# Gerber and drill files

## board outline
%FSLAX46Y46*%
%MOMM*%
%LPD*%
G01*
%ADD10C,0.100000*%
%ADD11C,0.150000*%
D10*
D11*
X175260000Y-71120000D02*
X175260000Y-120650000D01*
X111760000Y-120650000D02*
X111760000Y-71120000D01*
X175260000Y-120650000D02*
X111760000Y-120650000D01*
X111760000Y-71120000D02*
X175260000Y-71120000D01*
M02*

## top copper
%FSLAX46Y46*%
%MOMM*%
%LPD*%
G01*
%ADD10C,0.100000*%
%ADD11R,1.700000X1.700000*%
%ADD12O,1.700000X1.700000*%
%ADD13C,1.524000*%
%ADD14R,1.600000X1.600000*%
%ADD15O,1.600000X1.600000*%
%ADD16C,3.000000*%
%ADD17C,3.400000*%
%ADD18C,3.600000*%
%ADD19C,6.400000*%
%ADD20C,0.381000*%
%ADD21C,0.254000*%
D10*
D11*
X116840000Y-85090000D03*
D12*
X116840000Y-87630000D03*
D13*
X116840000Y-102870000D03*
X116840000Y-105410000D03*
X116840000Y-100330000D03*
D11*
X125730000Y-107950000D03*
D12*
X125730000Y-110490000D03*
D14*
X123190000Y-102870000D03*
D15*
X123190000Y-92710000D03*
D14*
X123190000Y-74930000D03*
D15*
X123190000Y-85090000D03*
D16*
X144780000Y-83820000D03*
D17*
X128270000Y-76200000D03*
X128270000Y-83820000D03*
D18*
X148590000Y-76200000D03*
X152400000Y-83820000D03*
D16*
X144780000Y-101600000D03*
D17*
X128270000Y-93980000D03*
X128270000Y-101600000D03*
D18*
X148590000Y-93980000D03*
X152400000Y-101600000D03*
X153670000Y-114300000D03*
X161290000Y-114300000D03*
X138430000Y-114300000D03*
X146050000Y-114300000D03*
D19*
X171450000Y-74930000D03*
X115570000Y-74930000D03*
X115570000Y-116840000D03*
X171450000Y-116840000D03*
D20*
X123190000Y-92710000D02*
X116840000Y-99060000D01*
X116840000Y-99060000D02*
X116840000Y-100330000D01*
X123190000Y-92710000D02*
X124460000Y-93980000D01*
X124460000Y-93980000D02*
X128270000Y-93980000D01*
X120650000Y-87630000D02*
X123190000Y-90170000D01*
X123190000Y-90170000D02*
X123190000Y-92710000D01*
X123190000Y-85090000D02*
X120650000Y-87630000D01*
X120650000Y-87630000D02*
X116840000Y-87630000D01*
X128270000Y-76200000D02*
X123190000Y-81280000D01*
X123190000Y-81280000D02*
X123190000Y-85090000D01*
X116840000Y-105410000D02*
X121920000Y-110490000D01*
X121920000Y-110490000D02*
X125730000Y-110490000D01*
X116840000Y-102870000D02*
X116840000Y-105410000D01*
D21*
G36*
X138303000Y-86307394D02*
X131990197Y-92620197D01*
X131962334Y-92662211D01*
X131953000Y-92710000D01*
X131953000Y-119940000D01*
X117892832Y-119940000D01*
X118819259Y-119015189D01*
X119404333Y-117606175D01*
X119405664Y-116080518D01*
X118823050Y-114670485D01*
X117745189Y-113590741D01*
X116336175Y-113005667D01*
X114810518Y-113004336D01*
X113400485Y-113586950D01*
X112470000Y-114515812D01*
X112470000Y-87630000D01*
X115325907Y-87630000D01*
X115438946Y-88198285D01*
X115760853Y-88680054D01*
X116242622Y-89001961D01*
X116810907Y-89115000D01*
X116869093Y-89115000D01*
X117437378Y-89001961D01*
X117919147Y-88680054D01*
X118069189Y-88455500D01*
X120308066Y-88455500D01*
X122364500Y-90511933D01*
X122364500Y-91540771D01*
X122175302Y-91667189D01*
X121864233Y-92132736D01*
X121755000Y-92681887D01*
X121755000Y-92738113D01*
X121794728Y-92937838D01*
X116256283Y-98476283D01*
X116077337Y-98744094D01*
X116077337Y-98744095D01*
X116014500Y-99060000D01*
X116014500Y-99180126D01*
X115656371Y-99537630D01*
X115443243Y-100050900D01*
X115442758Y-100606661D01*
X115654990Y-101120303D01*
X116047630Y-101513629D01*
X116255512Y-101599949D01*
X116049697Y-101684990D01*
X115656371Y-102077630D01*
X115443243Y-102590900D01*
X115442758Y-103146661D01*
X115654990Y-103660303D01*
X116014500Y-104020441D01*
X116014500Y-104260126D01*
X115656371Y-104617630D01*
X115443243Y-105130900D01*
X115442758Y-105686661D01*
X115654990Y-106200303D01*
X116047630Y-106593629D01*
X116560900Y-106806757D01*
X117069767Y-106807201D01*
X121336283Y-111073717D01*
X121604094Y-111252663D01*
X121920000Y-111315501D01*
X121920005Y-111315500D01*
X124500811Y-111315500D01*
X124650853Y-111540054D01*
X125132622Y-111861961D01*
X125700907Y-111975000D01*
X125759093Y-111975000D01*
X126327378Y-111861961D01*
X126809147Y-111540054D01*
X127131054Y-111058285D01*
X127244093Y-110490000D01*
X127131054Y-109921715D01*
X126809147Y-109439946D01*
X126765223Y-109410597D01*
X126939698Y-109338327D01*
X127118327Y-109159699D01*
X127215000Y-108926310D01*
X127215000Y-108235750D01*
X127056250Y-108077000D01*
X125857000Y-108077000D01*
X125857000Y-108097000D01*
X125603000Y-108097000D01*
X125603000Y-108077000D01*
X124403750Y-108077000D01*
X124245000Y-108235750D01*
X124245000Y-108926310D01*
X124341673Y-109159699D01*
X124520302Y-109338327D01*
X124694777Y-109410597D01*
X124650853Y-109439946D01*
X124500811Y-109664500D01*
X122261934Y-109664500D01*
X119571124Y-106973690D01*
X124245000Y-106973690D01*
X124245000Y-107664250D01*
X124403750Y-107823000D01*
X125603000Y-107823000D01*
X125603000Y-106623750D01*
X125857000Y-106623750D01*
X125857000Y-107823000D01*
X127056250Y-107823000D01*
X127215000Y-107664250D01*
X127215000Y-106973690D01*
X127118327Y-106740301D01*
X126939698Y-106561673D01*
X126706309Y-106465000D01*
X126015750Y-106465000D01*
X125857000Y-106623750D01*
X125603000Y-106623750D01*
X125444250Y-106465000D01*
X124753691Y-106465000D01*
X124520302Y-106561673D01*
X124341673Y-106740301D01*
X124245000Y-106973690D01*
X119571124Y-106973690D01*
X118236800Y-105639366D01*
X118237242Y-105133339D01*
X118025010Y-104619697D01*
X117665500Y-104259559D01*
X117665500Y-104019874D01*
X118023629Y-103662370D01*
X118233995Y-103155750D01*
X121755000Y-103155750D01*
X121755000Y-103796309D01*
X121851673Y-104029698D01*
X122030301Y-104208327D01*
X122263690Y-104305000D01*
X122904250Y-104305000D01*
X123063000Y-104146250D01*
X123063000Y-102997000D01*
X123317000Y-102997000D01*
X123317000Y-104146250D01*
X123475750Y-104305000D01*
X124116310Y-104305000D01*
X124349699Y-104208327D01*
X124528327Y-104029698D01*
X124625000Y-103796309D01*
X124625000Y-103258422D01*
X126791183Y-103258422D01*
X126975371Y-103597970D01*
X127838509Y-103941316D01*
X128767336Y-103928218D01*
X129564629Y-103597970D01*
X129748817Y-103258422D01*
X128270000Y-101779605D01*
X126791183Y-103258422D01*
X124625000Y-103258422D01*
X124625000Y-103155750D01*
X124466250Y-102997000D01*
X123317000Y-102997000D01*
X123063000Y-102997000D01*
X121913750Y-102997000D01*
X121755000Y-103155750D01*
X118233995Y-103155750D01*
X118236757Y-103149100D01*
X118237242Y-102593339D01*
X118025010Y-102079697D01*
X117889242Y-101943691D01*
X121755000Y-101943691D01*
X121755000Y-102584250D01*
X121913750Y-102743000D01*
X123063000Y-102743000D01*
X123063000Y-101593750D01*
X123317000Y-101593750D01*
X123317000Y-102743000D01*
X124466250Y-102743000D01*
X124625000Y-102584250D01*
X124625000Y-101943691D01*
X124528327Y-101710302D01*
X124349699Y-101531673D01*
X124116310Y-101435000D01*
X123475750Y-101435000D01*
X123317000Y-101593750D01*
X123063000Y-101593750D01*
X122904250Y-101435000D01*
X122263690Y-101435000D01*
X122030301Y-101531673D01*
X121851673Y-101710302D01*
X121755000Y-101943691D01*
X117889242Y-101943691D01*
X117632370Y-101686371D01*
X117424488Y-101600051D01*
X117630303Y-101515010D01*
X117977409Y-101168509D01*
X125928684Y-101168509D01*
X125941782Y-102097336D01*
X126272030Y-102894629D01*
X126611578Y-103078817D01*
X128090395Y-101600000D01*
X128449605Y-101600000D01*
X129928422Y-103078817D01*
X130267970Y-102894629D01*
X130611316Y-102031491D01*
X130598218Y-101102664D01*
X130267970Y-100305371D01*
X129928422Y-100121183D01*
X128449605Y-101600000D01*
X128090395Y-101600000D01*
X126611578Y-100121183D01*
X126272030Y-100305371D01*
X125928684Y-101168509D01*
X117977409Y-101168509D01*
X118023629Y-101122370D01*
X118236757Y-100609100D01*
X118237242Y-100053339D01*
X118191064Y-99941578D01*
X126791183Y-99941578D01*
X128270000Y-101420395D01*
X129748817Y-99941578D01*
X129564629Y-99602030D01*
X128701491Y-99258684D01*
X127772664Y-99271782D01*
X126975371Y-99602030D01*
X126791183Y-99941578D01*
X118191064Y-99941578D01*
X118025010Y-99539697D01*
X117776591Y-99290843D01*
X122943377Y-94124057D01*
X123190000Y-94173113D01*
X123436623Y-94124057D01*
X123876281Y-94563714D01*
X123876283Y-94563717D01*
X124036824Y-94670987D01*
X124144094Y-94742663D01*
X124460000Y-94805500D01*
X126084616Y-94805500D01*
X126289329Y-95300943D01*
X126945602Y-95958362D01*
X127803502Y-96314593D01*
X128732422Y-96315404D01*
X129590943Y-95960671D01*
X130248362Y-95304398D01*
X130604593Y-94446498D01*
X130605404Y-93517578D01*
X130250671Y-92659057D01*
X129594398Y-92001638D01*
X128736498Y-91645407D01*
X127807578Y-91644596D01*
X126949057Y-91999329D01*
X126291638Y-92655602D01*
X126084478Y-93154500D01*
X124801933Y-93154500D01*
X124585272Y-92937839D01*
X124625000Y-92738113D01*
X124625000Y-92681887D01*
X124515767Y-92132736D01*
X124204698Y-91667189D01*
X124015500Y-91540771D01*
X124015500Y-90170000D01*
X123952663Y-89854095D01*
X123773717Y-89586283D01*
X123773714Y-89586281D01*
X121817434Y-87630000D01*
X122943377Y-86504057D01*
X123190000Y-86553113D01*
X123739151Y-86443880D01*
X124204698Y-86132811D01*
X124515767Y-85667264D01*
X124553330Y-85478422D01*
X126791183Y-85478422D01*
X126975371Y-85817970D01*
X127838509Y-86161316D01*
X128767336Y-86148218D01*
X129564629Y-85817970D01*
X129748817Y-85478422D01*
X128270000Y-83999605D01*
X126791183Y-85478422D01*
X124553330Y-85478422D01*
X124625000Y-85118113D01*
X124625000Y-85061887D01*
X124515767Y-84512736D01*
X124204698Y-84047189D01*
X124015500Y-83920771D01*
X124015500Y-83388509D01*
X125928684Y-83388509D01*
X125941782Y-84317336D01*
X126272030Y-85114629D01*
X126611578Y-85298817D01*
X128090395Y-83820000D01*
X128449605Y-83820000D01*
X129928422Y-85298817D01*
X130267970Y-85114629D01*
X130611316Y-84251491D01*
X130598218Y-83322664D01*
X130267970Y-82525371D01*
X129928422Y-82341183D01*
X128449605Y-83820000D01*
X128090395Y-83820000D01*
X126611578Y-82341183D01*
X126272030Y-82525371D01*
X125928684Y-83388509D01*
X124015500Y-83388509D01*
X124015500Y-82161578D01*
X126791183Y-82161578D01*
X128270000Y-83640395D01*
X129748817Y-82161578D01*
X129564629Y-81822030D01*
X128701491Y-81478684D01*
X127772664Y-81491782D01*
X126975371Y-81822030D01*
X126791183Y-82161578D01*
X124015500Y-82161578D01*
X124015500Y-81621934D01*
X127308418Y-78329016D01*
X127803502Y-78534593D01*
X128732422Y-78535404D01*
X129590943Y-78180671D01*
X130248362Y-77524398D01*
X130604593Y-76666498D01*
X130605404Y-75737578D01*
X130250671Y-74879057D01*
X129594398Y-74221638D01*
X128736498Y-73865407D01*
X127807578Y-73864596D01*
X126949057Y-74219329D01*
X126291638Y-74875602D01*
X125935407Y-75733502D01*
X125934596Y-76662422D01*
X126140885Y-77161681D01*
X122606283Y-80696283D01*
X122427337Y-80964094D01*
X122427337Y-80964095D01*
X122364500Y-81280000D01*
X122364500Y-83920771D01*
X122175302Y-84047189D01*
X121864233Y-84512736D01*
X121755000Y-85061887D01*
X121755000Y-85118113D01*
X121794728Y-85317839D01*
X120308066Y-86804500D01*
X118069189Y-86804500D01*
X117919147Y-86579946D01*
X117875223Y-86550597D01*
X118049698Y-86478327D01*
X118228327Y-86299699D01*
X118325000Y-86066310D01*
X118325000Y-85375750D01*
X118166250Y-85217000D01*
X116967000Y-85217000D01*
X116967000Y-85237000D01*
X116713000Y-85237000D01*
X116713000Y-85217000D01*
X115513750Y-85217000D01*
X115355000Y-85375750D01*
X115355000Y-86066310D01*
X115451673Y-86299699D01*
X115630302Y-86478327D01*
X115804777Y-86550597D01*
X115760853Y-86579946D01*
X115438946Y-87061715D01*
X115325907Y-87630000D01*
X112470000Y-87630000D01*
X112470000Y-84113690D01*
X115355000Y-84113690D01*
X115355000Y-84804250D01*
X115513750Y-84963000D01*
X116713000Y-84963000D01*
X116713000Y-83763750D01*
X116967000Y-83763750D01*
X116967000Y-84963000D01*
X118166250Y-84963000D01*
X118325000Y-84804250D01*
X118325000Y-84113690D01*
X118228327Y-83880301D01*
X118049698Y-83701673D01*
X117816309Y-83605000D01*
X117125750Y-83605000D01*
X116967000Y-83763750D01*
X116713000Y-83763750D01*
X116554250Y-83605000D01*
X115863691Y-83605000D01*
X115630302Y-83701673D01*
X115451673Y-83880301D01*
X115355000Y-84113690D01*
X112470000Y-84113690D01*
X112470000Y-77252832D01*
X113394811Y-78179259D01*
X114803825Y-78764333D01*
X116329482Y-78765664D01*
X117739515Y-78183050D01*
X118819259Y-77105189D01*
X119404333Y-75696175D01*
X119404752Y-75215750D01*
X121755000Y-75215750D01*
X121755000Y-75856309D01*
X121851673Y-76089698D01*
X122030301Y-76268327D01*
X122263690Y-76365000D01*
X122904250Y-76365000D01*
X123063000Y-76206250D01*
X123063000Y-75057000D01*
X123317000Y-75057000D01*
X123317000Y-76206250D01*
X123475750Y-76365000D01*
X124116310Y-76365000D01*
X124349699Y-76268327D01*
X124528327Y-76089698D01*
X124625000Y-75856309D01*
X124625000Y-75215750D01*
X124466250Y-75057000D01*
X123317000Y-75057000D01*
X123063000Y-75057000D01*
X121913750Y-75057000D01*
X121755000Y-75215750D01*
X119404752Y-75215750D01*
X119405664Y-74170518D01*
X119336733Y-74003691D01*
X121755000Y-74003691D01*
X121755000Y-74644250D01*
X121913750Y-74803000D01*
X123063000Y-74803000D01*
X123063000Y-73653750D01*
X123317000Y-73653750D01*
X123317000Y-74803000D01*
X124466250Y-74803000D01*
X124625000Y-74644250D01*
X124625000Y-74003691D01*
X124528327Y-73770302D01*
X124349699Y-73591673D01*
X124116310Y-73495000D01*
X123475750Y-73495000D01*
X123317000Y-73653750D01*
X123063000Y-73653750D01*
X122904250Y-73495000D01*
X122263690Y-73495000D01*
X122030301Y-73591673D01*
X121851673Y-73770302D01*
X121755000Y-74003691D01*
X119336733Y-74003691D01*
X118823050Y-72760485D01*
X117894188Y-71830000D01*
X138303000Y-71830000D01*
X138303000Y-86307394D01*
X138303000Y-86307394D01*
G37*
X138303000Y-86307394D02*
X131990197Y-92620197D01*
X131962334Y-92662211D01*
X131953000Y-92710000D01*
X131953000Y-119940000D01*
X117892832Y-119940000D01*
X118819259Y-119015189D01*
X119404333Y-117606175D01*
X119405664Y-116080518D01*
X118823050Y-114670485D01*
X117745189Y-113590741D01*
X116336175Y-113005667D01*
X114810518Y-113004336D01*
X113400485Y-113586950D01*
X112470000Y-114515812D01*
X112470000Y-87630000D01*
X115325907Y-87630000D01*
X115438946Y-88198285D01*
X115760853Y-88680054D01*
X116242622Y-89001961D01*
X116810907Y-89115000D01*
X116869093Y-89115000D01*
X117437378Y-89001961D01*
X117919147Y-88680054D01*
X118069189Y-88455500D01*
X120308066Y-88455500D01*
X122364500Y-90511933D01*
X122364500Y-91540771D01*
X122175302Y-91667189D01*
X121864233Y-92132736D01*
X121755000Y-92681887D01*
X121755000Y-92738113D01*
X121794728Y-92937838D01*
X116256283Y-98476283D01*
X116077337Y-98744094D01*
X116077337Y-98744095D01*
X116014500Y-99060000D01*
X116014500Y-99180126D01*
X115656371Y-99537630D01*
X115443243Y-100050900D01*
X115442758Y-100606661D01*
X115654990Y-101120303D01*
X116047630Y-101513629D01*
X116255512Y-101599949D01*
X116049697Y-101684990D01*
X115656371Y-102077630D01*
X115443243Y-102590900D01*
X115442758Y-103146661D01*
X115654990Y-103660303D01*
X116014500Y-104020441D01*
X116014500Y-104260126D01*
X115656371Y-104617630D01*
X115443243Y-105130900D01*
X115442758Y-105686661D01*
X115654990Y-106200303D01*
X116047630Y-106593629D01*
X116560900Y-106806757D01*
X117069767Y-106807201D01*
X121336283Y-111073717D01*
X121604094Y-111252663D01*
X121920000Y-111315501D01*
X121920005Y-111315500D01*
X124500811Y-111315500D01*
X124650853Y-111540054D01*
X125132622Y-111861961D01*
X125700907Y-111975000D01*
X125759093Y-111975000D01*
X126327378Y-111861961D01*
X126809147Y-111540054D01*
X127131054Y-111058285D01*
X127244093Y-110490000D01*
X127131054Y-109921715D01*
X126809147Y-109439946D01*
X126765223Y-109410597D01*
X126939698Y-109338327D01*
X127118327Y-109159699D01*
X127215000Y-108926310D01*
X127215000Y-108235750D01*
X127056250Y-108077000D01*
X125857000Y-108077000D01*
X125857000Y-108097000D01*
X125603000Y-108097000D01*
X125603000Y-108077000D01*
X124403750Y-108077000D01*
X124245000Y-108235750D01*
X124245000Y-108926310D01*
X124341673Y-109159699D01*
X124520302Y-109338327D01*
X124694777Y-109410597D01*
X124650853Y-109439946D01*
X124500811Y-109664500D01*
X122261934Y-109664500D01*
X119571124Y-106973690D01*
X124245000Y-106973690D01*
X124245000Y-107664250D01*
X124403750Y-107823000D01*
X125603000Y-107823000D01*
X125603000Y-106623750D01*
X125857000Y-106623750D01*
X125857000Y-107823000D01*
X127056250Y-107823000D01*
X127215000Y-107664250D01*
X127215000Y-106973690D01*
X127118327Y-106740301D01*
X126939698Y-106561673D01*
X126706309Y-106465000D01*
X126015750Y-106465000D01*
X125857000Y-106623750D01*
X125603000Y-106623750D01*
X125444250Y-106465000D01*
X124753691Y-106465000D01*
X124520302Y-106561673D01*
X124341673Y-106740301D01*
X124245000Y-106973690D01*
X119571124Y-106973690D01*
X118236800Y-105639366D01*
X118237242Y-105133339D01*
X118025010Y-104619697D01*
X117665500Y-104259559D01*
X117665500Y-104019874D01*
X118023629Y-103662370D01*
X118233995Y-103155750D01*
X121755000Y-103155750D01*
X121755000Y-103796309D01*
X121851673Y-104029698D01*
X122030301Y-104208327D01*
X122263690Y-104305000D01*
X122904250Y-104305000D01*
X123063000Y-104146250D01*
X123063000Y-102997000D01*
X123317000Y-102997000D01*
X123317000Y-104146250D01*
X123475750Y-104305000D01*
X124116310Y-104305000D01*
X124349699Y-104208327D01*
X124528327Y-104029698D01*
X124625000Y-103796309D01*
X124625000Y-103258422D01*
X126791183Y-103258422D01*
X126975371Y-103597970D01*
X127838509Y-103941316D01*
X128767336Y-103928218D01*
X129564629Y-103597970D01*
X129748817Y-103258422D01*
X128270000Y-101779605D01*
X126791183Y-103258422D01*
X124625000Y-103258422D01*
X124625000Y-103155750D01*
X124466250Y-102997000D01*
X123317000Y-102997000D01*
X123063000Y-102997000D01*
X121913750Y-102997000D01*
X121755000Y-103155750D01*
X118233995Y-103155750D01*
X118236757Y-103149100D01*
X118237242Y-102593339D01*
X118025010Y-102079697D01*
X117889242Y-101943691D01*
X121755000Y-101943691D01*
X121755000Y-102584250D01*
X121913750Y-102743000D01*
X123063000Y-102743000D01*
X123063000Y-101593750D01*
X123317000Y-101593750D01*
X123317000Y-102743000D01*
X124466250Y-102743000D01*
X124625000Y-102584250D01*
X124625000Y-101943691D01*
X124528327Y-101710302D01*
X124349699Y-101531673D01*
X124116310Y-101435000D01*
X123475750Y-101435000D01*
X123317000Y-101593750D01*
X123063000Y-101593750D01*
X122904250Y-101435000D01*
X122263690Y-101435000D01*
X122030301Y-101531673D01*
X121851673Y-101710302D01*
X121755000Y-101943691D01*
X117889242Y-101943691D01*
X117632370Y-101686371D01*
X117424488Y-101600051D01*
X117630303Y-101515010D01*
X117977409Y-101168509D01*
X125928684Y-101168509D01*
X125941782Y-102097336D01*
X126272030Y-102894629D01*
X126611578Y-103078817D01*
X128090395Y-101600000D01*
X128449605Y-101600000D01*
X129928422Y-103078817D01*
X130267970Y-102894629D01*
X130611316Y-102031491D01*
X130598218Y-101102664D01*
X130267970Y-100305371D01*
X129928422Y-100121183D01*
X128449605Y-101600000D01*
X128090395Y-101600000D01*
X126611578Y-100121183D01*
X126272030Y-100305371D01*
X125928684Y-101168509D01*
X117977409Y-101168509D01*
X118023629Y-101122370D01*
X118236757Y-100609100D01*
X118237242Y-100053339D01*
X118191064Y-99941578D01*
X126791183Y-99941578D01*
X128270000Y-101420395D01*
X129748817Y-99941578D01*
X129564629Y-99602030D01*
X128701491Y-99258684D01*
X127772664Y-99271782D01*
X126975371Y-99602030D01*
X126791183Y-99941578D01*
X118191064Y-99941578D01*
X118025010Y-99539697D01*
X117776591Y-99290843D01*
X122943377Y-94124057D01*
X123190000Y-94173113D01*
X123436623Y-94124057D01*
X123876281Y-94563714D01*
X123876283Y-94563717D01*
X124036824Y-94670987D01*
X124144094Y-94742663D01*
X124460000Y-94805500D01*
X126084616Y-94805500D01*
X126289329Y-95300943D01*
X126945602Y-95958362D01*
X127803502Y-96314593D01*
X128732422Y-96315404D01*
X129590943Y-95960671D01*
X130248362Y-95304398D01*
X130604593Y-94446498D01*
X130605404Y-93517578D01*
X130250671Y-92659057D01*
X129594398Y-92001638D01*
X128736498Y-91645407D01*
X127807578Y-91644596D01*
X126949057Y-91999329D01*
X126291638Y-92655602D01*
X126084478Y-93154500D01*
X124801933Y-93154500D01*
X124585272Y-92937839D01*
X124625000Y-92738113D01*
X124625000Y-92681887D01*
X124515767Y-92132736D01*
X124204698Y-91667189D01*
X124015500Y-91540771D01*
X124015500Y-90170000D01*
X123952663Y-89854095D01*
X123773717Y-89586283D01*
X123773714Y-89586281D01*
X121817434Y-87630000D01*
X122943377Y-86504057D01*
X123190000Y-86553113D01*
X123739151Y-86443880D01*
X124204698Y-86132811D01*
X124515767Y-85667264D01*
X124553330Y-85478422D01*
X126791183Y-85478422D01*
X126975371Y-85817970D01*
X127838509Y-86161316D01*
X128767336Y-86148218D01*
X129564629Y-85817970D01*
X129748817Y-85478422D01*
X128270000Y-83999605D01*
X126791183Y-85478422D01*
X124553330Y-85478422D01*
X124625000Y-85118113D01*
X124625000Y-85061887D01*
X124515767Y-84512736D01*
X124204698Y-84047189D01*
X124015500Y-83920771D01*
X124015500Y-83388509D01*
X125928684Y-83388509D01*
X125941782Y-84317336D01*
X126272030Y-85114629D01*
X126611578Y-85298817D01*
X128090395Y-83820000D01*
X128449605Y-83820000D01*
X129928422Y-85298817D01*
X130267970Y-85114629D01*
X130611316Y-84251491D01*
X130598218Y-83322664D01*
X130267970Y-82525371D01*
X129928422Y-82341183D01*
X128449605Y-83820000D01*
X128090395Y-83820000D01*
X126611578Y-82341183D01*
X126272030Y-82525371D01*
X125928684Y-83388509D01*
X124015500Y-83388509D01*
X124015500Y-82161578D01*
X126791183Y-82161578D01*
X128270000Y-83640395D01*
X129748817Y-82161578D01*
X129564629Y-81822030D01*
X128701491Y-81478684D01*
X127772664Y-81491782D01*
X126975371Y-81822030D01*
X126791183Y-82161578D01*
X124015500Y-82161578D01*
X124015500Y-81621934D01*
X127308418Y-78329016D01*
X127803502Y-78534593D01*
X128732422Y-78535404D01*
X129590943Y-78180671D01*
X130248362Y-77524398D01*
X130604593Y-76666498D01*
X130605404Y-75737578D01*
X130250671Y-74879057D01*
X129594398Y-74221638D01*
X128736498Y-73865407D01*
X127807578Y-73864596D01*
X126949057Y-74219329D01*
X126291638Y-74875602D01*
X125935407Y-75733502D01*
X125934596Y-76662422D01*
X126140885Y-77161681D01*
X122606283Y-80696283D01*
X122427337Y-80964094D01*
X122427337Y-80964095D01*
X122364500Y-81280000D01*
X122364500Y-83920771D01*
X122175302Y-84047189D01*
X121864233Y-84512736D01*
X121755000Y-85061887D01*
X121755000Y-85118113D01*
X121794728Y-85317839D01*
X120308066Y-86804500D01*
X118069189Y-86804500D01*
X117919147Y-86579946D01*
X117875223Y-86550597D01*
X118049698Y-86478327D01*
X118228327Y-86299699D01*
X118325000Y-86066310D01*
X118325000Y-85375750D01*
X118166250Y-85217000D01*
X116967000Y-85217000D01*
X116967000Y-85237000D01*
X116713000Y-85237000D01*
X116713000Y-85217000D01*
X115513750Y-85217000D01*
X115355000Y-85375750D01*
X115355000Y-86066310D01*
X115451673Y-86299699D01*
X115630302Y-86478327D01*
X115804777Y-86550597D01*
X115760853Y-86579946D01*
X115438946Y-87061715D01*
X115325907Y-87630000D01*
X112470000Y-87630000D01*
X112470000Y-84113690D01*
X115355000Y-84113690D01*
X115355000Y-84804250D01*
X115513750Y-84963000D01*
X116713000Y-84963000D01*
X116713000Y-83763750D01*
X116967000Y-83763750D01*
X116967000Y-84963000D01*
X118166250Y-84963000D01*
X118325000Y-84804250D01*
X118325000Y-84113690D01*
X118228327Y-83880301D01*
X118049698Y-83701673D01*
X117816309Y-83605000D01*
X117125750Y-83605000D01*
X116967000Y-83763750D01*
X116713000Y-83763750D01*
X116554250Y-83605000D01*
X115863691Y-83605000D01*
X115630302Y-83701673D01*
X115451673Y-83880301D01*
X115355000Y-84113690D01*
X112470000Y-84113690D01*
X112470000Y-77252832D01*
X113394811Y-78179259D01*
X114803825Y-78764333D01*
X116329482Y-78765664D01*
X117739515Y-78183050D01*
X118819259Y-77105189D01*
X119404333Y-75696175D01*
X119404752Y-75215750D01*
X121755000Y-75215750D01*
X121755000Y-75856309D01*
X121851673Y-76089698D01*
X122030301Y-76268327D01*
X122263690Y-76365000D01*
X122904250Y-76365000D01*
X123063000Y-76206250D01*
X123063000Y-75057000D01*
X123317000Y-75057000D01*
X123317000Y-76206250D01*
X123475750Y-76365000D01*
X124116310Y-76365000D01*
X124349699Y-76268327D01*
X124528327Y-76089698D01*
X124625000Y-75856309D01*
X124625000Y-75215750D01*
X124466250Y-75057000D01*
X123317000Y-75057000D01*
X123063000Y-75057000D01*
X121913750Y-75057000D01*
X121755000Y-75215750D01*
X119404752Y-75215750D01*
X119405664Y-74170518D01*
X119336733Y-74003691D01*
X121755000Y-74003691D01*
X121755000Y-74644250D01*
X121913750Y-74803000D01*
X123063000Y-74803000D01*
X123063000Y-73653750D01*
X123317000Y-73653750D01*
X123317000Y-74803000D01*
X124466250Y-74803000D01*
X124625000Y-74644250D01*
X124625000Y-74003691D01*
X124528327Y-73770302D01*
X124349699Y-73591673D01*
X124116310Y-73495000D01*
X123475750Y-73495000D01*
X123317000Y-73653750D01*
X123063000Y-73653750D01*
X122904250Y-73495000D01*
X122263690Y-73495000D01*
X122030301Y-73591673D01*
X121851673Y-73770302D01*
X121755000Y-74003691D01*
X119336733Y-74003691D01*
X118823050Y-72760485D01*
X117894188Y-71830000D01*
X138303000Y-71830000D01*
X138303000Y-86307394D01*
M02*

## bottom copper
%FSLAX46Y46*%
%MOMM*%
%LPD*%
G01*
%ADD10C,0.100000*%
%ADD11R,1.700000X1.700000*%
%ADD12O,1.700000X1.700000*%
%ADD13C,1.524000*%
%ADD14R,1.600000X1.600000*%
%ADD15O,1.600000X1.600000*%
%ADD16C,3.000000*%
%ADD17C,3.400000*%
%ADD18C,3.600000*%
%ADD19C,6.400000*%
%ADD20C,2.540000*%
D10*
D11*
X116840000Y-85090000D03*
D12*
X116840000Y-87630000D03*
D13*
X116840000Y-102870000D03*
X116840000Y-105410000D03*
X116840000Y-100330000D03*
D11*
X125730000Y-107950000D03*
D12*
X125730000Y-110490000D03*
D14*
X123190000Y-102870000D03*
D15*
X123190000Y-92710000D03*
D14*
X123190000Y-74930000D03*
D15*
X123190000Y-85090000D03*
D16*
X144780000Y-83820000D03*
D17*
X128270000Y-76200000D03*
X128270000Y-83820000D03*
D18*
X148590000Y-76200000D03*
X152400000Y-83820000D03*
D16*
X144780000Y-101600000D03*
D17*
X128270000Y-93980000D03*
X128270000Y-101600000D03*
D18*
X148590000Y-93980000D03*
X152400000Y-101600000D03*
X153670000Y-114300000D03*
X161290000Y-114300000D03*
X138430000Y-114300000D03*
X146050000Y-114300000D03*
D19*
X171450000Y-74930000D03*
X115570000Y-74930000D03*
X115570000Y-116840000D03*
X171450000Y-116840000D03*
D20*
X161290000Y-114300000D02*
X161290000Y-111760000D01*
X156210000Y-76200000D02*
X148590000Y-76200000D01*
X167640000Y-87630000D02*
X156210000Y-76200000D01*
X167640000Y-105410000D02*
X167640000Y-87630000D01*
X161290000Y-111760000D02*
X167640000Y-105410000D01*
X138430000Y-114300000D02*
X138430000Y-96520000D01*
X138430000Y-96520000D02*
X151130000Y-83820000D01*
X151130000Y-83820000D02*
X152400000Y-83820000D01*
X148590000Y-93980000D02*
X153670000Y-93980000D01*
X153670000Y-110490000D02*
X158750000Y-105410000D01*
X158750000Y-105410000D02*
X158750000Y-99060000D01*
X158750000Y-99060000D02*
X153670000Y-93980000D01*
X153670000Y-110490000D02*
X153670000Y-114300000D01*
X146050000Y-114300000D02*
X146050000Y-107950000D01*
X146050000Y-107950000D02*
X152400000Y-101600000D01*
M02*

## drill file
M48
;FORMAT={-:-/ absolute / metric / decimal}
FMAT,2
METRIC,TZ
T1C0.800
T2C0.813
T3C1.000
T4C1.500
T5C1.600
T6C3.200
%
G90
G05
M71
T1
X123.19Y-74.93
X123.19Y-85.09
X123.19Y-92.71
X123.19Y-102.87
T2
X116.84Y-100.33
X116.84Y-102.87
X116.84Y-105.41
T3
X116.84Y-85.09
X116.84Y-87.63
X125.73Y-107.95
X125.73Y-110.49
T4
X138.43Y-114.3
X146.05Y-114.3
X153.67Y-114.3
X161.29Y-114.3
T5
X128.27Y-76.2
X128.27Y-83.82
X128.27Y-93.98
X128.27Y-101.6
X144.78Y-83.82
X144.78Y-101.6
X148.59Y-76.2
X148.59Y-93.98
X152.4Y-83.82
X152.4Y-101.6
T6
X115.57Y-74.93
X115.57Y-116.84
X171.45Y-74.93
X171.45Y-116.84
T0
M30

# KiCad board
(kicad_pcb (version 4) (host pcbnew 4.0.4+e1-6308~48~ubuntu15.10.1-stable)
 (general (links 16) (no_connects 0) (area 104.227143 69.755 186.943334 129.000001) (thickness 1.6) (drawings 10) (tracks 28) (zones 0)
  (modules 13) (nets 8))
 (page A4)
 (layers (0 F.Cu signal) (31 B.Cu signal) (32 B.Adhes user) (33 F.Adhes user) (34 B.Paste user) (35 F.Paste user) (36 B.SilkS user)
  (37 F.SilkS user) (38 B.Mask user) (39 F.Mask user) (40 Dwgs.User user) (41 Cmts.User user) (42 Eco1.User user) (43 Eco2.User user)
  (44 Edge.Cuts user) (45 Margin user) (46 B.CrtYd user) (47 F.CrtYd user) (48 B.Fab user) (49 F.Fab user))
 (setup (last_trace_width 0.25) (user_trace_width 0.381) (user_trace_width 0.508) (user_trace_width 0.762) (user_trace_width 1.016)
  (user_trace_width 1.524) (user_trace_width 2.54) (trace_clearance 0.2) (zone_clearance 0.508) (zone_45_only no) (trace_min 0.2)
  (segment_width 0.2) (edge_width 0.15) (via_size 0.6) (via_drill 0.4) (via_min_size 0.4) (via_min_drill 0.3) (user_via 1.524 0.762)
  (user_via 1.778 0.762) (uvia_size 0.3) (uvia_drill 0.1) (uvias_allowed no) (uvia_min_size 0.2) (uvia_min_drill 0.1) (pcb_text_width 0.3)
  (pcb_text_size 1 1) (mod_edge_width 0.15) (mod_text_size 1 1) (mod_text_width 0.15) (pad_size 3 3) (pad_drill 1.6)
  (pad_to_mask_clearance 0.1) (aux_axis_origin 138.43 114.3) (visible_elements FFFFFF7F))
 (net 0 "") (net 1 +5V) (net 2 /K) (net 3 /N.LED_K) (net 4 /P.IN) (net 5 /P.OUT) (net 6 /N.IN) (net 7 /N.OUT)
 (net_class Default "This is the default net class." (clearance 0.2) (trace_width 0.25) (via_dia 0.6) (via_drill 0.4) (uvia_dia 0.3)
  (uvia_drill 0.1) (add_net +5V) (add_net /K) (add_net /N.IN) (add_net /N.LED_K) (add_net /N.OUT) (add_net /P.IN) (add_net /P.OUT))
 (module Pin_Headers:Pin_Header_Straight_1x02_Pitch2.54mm (layer F.Cu) (at 116.84 85.09)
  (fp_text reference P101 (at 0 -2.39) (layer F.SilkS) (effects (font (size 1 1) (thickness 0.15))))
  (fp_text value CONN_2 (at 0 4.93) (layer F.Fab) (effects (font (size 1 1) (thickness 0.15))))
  (pad 1 thru_hole rect (at 0 0) (size 1.7 1.7) (drill 1) (layers *.Cu *.Mask) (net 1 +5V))
  (pad 2 thru_hole oval (at 0 2.54) (size 1.7 1.7) (drill 1) (layers *.Cu *.Mask) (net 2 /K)))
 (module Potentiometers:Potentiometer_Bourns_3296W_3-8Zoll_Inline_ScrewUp (layer F.Cu) (at 116.84 100.33 180)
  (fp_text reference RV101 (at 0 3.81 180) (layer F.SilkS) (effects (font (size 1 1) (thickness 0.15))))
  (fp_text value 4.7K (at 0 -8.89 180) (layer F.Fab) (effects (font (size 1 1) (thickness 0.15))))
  (pad 2 thru_hole circle (at 0 -2.54 180) (size 1.524 1.524) (drill 0.8128) (layers *.Cu *.Mask) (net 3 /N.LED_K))
  (pad 3 thru_hole circle (at 0 -5.08 180) (size 1.524 1.524) (drill 0.8128) (layers *.Cu *.Mask) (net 3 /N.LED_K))
  (pad 1 thru_hole circle (at 0 0 180) (size 1.524 1.524) (drill 0.8128) (layers *.Cu *.Mask) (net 2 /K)))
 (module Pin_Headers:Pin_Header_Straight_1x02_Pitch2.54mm (layer F.Cu) (at 125.73 107.95)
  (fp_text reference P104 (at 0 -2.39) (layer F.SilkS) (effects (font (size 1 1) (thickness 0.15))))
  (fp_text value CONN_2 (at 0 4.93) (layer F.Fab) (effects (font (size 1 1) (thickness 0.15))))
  (pad 1 thru_hole rect (at 0 0) (size 1.7 1.7) (drill 1) (layers *.Cu *.Mask) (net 1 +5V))
  (pad 2 thru_hole oval (at 0 2.54) (size 1.7 1.7) (drill 1) (layers *.Cu *.Mask) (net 3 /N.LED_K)))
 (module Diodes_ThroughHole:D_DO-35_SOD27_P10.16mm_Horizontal (layer F.Cu) (at 123.19 102.87 90)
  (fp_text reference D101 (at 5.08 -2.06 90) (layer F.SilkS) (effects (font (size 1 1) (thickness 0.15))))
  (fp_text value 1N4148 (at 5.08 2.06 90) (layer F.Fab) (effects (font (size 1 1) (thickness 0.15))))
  (pad 1 thru_hole rect (at 0 0 90) (size 1.6 1.6) (drill 0.8) (layers *.Cu *.Mask) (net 1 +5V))
  (pad 2 thru_hole oval (at 10.16 0 90) (size 1.6 1.6) (drill 0.8) (layers *.Cu *.Mask) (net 2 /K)))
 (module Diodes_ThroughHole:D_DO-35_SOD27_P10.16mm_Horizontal (layer F.Cu) (at 123.19 74.93 270)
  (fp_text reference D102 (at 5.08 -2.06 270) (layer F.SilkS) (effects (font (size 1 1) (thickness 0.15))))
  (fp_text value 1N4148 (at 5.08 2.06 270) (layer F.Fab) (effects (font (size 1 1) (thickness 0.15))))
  (pad 1 thru_hole rect (at 0 0 270) (size 1.6 1.6) (drill 0.8) (layers *.Cu *.Mask) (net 1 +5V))
  (pad 2 thru_hole oval (at 10.16 0 270) (size 1.6 1.6) (drill 0.8) (layers *.Cu *.Mask) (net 2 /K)))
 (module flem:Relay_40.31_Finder (layer F.Cu) (at 128.27 83.82)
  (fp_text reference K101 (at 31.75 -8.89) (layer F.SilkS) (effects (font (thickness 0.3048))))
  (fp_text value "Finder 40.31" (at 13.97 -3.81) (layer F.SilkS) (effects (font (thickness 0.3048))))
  (pad 12 thru_hole circle (at 16.51 0) (size 3 3) (drill 1.6) (layers *.Cu *.Mask F.SilkS))
  (pad A2 thru_hole circle (at 0 -7.62) (size 3.4 3.4) (drill 1.6) (layers *.Cu *.Mask F.SilkS) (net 2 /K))
  (pad A1 thru_hole circle (at 0 0) (size 3.4 3.4) (drill 1.6) (layers *.Cu *.Mask F.SilkS) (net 1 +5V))
  (pad 11 thru_hole circle (at 20.32 -7.62) (size 3.6 3.6) (drill 1.6) (layers *.Cu *.Mask F.SilkS) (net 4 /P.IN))
  (pad 14 thru_hole circle (at 24.13 0) (size 3.6 3.6) (drill 1.6) (layers *.Cu *.Mask F.SilkS) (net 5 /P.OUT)))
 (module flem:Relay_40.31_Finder (layer F.Cu) (at 128.27 101.6)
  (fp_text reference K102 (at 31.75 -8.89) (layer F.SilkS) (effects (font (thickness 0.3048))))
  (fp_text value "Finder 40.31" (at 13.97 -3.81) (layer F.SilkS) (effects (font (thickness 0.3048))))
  (pad 12 thru_hole circle (at 16.51 0) (size 3 3) (drill 1.6) (layers *.Cu *.Mask F.SilkS))
  (pad A2 thru_hole circle (at 0 -7.62) (size 3.4 3.4) (drill 1.6) (layers *.Cu *.Mask F.SilkS) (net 2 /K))
  (pad A1 thru_hole circle (at 0 0) (size 3.4 3.4) (drill 1.6) (layers *.Cu *.Mask F.SilkS) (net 1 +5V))
  (pad 11 thru_hole circle (at 20.32 -7.62) (size 3.6 3.6) (drill 1.6) (layers *.Cu *.Mask F.SilkS) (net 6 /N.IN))
  (pad 14 thru_hole circle (at 24.13 0) (size 3.6 3.6) (drill 1.6) (layers *.Cu *.Mask F.SilkS) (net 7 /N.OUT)))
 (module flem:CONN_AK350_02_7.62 (layer F.Cu) (at 153.67 114.3)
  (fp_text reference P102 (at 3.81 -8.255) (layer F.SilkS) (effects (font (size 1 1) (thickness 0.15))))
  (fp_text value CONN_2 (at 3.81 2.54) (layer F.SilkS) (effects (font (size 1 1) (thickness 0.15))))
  (pad 1 thru_hole circle (at 0 0) (size 3.6 3.6) (drill 1.5) (layers *.Cu *.Mask) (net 6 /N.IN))
  (pad 2 thru_hole circle (at 7.62 0) (size 3.6 3.6) (drill 1.5) (layers *.Cu *.Mask) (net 4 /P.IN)))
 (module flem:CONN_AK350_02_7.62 (layer F.Cu) (at 138.43 114.3)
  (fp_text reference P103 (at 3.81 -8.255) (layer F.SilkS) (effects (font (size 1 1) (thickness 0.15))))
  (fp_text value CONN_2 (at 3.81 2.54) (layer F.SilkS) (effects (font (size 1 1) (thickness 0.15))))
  (pad 1 thru_hole circle (at 0 0) (size 3.6 3.6) (drill 1.5) (layers *.Cu *.Mask) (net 5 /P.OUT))
  (pad 2 thru_hole circle (at 7.62 0) (size 3.6 3.6) (drill 1.5) (layers *.Cu *.Mask) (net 7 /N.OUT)))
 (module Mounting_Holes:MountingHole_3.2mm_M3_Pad (layer F.Cu) (at 171.45 74.93)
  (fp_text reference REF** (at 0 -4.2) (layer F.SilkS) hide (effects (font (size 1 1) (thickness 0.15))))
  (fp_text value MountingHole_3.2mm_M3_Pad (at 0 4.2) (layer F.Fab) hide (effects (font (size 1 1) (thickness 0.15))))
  (pad 1 thru_hole circle (at 0 0) (size 6.4 6.4) (drill 3.2) (layers *.Cu *.Mask)))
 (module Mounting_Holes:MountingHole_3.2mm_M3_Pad (layer F.Cu) (at 115.57 74.93)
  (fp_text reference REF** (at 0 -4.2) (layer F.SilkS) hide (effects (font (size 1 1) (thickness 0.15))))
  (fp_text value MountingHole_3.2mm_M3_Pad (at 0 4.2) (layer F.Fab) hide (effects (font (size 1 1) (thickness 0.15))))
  (pad 1 thru_hole circle (at 0 0) (size 6.4 6.4) (drill 3.2) (layers *.Cu *.Mask)))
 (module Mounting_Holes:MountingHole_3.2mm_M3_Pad (layer F.Cu) (at 115.57 116.84)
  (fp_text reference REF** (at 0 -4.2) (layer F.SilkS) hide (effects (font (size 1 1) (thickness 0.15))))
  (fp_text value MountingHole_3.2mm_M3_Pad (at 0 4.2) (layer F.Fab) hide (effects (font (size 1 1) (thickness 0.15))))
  (pad 1 thru_hole circle (at 0 0) (size 6.4 6.4) (drill 3.2) (layers *.Cu *.Mask)))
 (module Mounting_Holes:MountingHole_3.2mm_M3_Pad (layer F.Cu) (at 171.45 116.84)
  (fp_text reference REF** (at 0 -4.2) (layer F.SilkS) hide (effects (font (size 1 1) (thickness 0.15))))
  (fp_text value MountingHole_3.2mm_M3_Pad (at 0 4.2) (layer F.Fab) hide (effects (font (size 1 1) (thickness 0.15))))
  (pad 1 thru_hole circle (at 0 0) (size 6.4 6.4) (drill 3.2) (layers *.Cu *.Mask)))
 (gr_line (start 175.26 71.12) (end 175.26 120.65) (angle 90) (layer Edge.Cuts) (width 0.15))
 (gr_line (start 111.76 120.65) (end 111.76 71.12) (angle 90) (layer Edge.Cuts) (width 0.15))
 (gr_line (start 175.26 120.65) (end 111.76 120.65) (angle 90) (layer Edge.Cuts) (width 0.15))
 (gr_line (start 111.76 71.12) (end 175.26 71.12) (angle 90) (layer Edge.Cuts) (width 0.15))
 (segment (start 123.19 92.71) (end 116.84 99.06) (width 0.381) (layer F.Cu) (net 2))
 (segment (start 116.84 99.06) (end 116.84 100.33) (width 0.381) (layer F.Cu) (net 2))
 (segment (start 123.19 92.71) (end 124.46 93.98) (width 0.381) (layer F.Cu) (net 2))
 (segment (start 124.46 93.98) (end 128.27 93.98) (width 0.381) (layer F.Cu) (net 2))
 (segment (start 120.65 87.63) (end 123.19 90.17) (width 0.381) (layer F.Cu) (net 2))
 (segment (start 123.19 90.17) (end 123.19 92.71) (width 0.381) (layer F.Cu) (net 2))
 (segment (start 123.19 85.09) (end 120.65 87.63) (width 0.381) (layer F.Cu) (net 2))
 (segment (start 120.65 87.63) (end 116.84 87.63) (width 0.381) (layer F.Cu) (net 2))
 (segment (start 128.27 76.2) (end 123.19 81.28) (width 0.381) (layer F.Cu) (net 2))
 (segment (start 123.19 81.28) (end 123.19 85.09) (width 0.381) (layer F.Cu) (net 2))
 (segment (start 161.29 114.3) (end 161.29 111.76) (width 2.54) (layer B.Cu) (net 4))
 (segment (start 156.21 76.2) (end 148.59 76.2) (width 2.54) (layer B.Cu) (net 4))
 (segment (start 167.64 87.63) (end 156.21 76.2) (width 2.54) (layer B.Cu) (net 4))
 (segment (start 167.64 105.41) (end 167.64 87.63) (width 2.54) (layer B.Cu) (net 4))
 (segment (start 161.29 111.76) (end 167.64 105.41) (width 2.54) (layer B.Cu) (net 4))
 (segment (start 138.43 114.3) (end 138.43 96.52) (width 2.54) (layer B.Cu) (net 5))
 (segment (start 138.43 96.52) (end 151.13 83.82) (width 2.54) (layer B.Cu) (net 5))
 (segment (start 151.13 83.82) (end 152.4 83.82) (width 2.54) (layer B.Cu) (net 5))
 (segment (start 148.59 93.98) (end 153.67 93.98) (width 2.54) (layer B.Cu) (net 6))
 (segment (start 153.67 110.49) (end 158.75 105.41) (width 2.54) (layer B.Cu) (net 6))
 (segment (start 158.75 105.41) (end 158.75 99.06) (width 2.54) (layer B.Cu) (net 6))
 (segment (start 158.75 99.06) (end 153.67 93.98) (width 2.54) (layer B.Cu) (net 6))
 (segment (start 153.67 110.49) (end 153.67 114.3) (width 2.54) (layer B.Cu) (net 6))
 (segment (start 146.05 114.3) (end 146.05 107.95) (width 2.54) (layer B.Cu) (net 7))
 (segment (start 146.05 107.95) (end 152.4 101.6) (width 2.54) (layer B.Cu) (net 7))
 (segment (start 116.84 105.41) (end 121.92 110.49) (width 0.381) (layer F.Cu) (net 3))
 (segment (start 121.92 110.49) (end 125.73 110.49) (width 0.381) (layer F.Cu) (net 3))
 (segment (start 116.84 102.87) (end 116.84 105.41) (width 0.381) (layer F.Cu) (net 3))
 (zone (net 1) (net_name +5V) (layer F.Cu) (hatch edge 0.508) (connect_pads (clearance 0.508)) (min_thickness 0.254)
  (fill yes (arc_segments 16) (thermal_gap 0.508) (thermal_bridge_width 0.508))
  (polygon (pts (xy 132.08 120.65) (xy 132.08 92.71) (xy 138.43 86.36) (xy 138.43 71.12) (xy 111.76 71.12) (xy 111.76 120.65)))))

